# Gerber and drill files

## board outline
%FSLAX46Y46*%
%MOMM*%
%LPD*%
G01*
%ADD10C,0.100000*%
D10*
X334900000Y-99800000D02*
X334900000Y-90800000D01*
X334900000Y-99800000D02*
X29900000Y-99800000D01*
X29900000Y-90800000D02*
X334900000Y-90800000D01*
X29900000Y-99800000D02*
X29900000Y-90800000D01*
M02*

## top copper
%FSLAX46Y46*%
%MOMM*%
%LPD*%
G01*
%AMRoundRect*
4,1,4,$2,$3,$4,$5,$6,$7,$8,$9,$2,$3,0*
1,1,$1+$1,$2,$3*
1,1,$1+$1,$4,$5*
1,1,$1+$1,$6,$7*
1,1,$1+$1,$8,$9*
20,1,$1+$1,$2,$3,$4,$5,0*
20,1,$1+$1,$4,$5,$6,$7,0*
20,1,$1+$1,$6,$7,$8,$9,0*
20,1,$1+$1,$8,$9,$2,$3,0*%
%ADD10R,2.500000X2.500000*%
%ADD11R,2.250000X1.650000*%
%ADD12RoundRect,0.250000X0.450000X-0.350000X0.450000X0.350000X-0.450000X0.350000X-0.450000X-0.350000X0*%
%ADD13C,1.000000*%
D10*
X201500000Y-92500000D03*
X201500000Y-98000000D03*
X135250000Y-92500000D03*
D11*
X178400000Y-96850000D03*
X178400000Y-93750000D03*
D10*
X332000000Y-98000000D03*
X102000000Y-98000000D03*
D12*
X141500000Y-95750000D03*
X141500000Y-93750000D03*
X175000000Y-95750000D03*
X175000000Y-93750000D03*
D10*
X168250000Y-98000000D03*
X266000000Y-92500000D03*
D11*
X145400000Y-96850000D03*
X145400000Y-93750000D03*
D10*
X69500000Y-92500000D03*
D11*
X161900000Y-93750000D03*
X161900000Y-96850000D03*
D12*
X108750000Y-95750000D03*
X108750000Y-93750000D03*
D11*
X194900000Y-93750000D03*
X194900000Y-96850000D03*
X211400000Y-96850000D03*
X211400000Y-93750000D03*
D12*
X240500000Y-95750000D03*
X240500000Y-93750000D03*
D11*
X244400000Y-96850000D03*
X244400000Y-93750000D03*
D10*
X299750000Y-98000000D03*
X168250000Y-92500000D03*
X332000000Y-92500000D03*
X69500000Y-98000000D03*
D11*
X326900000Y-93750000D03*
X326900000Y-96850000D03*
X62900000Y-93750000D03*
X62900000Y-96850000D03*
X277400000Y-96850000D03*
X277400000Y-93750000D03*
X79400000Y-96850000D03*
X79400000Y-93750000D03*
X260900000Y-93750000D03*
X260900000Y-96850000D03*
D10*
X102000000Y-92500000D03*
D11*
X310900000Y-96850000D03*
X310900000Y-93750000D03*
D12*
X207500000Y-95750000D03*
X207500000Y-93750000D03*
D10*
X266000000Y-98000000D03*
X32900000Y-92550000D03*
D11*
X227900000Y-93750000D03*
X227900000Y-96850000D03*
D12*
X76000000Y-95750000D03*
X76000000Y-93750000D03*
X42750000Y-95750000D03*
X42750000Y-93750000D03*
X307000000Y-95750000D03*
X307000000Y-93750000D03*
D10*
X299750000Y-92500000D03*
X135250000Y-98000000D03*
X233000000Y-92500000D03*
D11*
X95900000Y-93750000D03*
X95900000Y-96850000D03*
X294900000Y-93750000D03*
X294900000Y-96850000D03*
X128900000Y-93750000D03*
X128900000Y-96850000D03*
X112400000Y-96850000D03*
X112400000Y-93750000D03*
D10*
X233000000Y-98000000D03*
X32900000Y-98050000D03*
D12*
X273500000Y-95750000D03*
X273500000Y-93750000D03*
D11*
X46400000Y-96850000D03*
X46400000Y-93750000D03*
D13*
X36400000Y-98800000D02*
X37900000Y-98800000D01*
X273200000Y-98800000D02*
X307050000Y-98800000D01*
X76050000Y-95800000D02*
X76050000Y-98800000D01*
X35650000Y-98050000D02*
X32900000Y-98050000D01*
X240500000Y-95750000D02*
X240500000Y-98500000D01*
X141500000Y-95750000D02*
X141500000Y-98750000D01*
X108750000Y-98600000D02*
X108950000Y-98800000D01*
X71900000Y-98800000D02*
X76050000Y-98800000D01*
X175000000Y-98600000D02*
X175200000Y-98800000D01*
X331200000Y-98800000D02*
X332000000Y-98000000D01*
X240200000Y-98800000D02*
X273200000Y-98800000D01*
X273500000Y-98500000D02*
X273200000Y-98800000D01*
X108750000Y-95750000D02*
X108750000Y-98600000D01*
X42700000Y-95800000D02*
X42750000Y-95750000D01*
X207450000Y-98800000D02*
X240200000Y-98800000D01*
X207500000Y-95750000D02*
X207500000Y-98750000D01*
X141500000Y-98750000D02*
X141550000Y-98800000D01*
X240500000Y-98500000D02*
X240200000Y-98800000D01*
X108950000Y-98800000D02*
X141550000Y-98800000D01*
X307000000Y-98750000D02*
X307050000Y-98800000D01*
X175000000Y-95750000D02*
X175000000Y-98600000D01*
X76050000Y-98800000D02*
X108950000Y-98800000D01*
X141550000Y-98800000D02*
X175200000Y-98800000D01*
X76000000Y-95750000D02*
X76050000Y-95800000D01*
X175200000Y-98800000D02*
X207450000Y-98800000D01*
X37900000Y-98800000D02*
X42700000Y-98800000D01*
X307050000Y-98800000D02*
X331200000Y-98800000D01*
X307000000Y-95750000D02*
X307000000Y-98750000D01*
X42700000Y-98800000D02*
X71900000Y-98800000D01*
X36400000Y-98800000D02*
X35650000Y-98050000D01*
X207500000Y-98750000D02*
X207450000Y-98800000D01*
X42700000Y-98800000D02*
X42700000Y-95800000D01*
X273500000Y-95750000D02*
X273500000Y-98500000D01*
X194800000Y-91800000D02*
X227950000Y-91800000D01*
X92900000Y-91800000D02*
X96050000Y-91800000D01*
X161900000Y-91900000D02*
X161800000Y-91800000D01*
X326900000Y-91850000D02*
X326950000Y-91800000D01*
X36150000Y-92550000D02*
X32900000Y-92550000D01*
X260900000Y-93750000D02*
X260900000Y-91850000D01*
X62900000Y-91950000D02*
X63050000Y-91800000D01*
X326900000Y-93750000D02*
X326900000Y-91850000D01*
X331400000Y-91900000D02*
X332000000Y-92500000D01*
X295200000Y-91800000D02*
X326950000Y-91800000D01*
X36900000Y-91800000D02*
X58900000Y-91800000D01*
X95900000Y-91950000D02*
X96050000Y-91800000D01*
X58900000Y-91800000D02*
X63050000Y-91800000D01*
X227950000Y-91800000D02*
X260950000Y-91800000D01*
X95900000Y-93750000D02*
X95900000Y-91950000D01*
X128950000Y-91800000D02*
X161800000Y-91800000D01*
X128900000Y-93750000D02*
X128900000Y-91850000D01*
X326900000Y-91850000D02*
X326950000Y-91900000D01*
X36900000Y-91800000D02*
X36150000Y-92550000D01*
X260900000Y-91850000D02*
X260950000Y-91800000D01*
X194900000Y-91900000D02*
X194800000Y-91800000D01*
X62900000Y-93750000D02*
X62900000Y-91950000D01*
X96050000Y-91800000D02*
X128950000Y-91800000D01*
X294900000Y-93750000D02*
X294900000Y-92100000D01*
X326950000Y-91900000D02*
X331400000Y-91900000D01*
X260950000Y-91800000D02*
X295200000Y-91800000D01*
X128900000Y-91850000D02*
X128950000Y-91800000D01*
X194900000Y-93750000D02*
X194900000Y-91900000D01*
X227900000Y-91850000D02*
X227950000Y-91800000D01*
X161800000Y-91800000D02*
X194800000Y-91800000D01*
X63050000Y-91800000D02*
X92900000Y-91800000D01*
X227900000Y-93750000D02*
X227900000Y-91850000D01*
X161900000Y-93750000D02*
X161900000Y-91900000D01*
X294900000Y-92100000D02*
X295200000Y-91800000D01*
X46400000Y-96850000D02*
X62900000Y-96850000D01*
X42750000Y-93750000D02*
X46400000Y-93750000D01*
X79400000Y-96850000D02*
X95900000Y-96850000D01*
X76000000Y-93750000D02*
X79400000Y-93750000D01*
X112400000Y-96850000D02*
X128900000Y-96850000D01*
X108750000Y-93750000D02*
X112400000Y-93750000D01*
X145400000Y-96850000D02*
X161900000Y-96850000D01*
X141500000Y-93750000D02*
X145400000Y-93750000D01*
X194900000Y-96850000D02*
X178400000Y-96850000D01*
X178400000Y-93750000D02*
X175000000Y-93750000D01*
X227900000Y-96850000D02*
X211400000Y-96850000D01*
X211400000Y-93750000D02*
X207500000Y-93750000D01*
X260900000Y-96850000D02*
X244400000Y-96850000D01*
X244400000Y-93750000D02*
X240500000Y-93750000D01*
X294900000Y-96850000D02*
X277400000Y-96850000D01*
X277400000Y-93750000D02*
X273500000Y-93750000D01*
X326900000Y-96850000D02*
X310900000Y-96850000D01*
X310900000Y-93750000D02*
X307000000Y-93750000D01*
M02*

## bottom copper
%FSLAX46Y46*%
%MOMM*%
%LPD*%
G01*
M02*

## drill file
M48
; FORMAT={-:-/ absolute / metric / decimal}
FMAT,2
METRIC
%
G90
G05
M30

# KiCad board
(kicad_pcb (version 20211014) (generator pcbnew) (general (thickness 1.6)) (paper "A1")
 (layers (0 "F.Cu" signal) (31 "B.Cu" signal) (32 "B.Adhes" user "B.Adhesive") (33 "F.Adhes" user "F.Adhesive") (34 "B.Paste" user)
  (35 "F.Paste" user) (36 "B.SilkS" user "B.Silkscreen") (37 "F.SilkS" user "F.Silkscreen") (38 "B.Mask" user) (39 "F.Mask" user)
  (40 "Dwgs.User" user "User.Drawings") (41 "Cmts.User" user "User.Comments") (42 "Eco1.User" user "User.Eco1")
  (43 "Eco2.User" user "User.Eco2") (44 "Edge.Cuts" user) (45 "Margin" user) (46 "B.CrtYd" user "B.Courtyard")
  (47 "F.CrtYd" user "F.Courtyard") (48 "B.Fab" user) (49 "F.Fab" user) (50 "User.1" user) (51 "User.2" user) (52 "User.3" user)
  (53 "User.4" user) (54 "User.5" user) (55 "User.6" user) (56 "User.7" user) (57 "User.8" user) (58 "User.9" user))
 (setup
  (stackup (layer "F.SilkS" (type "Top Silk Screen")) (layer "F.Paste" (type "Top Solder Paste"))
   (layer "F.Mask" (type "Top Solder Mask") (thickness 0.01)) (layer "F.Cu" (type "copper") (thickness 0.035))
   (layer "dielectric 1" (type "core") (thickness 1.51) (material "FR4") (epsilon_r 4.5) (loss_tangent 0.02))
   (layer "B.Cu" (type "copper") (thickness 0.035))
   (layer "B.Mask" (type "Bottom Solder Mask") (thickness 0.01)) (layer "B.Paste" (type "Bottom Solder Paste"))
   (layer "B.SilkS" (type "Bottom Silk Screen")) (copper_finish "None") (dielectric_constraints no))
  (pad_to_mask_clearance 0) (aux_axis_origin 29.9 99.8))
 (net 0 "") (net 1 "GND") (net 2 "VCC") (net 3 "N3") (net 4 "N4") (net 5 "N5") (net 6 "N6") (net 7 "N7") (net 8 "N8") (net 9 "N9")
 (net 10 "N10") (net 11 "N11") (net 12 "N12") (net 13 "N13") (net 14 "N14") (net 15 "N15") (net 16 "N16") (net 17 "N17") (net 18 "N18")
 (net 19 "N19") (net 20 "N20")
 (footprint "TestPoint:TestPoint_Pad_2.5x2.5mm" (layer "F.Cu") (at 201.5 92.5)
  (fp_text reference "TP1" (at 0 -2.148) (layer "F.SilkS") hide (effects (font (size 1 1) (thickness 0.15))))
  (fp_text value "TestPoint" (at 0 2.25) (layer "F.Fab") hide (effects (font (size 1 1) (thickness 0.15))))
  (pad "1" smd rect (at 0 0) (size 2.5 2.5) (layers "F.Cu" "F.Mask") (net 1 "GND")))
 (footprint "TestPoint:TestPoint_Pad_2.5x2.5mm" (layer "F.Cu") (at 201.5 98)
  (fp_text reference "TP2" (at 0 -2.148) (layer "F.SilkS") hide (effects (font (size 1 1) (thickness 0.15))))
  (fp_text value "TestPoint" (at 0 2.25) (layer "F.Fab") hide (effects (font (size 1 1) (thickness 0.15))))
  (pad "1" smd rect (at 0 0) (size 2.5 2.5) (layers "F.Cu" "F.Mask") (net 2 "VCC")))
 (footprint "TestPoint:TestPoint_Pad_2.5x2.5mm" (layer "F.Cu") (at 135.25 92.5)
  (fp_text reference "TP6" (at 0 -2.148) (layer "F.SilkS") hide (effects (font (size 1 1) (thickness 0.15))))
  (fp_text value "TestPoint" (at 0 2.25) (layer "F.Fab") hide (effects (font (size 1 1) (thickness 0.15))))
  (pad "1" smd rect (at 0 0) (size 2.5 2.5) (layers "F.Cu" "F.Mask") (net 1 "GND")))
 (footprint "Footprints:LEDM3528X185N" (layer "F.Cu") (at 178.4 95.3 90)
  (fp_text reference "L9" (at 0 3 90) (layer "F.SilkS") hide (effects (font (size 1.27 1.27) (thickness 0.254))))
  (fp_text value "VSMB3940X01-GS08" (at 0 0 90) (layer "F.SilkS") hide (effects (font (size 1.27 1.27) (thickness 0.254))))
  (pad "1" smd rect (at -1.55 0 90) (size 1.65 2.25) (layers "F.Cu" "F.Paste" "F.Mask") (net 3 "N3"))
  (pad "2" smd rect (at 1.55 0 90) (size 1.65 2.25) (layers "F.Cu" "F.Paste" "F.Mask") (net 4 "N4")))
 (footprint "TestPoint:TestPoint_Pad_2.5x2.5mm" (layer "F.Cu") (at 332 98)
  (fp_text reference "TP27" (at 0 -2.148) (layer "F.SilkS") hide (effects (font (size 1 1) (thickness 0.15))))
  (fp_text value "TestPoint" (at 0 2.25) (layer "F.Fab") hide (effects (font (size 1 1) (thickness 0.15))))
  (pad "1" smd rect (at 0 0) (size 2.5 2.5) (layers "F.Cu" "F.Mask") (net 2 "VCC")))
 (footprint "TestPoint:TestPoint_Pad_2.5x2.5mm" (layer "F.Cu") (at 102 98)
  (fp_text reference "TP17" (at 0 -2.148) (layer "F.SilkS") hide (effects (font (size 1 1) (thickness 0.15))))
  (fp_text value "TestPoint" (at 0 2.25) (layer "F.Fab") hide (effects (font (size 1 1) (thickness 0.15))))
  (pad "1" smd rect (at 0 0) (size 2.5 2.5) (layers "F.Cu" "F.Mask") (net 2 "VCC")))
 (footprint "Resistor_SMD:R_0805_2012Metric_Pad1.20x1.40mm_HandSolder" (layer "F.Cu") (at 141.5 94.75 90)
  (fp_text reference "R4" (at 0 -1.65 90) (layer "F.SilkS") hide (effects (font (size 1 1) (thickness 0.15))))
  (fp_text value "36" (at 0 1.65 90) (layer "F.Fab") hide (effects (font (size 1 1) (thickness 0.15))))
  (pad "1" smd roundrect (at -1 0 90) (size 1.2 1.4) (layers "F.Cu" "F.Paste" "F.Mask") (roundrect_rratio 0.2083333333) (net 2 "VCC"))
  (pad "2" smd roundrect (at 1 0 90) (size 1.2 1.4) (layers "F.Cu" "F.Paste" "F.Mask") (roundrect_rratio 0.2083333333) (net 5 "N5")))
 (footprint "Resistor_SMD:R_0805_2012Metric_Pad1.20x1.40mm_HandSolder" (layer "F.Cu") (at 175 94.75 90)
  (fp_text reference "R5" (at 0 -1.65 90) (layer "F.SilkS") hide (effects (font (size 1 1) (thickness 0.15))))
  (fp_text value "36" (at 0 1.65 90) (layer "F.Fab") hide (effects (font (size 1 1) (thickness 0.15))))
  (pad "1" smd roundrect (at -1 0 90) (size 1.2 1.4) (layers "F.Cu" "F.Paste" "F.Mask") (roundrect_rratio 0.2083333333) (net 2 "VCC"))
  (pad "2" smd roundrect (at 1 0 90) (size 1.2 1.4) (layers "F.Cu" "F.Paste" "F.Mask") (roundrect_rratio 0.2083333333) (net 4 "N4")))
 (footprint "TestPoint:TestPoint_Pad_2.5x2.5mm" (layer "F.Cu") (at 168.25 98)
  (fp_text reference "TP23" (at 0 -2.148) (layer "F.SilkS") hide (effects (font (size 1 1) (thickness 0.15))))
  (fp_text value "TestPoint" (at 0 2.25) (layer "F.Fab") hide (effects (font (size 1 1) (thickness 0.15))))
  (pad "1" smd rect (at 0 0) (size 2.5 2.5) (layers "F.Cu" "F.Mask") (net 2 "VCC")))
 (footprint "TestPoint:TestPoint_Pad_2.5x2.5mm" (layer "F.Cu") (at 266 92.5)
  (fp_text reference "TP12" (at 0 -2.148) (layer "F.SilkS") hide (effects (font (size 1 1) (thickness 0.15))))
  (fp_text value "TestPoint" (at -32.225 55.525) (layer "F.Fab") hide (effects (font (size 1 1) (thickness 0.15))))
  (pad "1" smd rect (at 0 0) (size 2.5 2.5) (layers "F.Cu" "F.Mask") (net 1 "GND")))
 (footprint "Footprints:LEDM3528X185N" (layer "F.Cu") (at 145.4 95.3 90)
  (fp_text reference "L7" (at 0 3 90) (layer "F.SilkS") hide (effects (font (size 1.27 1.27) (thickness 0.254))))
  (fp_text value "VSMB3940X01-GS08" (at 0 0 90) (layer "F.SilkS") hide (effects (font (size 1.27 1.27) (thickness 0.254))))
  (pad "1" smd rect (at -1.55 0 90) (size 1.65 2.25) (layers "F.Cu" "F.Paste" "F.Mask") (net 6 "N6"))
  (pad "2" smd rect (at 1.55 0 90) (size 1.65 2.25) (layers "F.Cu" "F.Paste" "F.Mask") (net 5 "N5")))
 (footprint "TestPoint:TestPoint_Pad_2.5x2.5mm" (layer "F.Cu") (at 69.5 92.5)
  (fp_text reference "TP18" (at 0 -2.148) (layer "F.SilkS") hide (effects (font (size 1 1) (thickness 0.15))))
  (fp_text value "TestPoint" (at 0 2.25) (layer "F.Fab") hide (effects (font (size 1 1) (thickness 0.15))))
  (pad "1" smd rect (at 0 0) (size 2.5 2.5) (layers "F.Cu" "F.Mask") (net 1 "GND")))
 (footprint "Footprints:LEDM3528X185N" (layer "F.Cu") (at 161.9 95.3 -90)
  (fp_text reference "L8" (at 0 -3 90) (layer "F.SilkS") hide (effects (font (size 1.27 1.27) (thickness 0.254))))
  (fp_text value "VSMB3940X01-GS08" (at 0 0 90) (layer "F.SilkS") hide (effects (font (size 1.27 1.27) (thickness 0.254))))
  (pad "1" smd rect (at -1.55 0 270) (size 1.65 2.25) (layers "F.Cu" "F.Paste" "F.Mask") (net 1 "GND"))
  (pad "2" smd rect (at 1.55 0 270) (size 1.65 2.25) (layers "F.Cu" "F.Paste" "F.Mask") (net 6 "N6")))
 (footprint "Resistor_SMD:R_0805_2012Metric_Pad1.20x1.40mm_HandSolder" (layer "F.Cu") (at 108.75 94.75 90)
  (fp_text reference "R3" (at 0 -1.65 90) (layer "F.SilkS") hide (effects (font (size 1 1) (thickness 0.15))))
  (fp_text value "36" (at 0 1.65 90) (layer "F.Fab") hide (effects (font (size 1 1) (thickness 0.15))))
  (pad "1" smd roundrect (at -1 0 90) (size 1.2 1.4) (layers "F.Cu" "F.Paste" "F.Mask") (roundrect_rratio 0.2083333333) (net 2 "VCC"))
  (pad "2" smd roundrect (at 1 0 90) (size 1.2 1.4) (layers "F.Cu" "F.Paste" "F.Mask") (roundrect_rratio 0.2083333333) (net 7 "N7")))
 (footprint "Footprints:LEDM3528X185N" (layer "F.Cu") (at 194.9 95.3 -90)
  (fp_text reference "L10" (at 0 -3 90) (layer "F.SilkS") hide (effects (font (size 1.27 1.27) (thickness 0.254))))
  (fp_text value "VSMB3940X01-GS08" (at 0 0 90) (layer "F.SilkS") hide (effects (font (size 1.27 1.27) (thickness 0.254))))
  (pad "1" smd rect (at -1.55 0 270) (size 1.65 2.25) (layers "F.Cu" "F.Paste" "F.Mask") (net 1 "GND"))
  (pad "2" smd rect (at 1.55 0 270) (size 1.65 2.25) (layers "F.Cu" "F.Paste" "F.Mask") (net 3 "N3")))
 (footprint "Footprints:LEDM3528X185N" (layer "F.Cu") (at 211.4 95.3 90)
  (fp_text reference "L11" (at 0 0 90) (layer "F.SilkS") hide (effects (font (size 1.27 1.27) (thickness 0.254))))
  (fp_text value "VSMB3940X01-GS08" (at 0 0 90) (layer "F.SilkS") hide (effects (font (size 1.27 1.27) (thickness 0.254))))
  (pad "1" smd rect (at -1.55 0 90) (size 1.65 2.25) (layers "F.Cu" "F.Paste" "F.Mask") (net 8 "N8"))
  (pad "2" smd rect (at 1.55 0 90) (size 1.65 2.25) (layers "F.Cu" "F.Paste" "F.Mask") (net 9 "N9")))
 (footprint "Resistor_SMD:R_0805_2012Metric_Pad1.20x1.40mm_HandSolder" (layer "F.Cu") (at 240.5 94.75 90)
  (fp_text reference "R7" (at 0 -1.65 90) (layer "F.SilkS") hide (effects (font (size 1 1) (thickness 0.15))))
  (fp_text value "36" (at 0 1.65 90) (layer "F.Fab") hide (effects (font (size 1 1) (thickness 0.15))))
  (pad "1" smd roundrect (at -1 0 90) (size 1.2 1.4) (layers "F.Cu" "F.Paste" "F.Mask") (roundrect_rratio 0.2083333333) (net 2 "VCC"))
  (pad "2" smd roundrect (at 1 0 90) (size 1.2 1.4) (layers "F.Cu" "F.Paste" "F.Mask") (roundrect_rratio 0.2083333333) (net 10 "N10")))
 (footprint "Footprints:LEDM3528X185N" (layer "F.Cu") (at 244.4 95.3 90)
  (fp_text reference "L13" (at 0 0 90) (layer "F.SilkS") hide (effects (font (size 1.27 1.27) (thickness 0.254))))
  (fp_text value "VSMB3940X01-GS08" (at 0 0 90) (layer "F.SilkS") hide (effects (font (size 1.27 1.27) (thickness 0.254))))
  (pad "1" smd rect (at -1.55 0 90) (size 1.65 2.25) (layers "F.Cu" "F.Paste" "F.Mask") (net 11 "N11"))
  (pad "2" smd rect (at 1.55 0 90) (size 1.65 2.25) (layers "F.Cu" "F.Paste" "F.Mask") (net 10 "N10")))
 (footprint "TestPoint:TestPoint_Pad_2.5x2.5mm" (layer "F.Cu") (at 299.75 98)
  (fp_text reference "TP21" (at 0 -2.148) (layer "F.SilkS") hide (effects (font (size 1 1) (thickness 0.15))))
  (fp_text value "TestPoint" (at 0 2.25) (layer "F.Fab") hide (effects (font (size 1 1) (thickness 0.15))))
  (pad "1" smd rect (at 0 0) (size 2.5 2.5) (layers "F.Cu" "F.Mask") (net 2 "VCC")))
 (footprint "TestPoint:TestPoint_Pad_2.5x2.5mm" (layer "F.Cu") (at 168.25 92.5)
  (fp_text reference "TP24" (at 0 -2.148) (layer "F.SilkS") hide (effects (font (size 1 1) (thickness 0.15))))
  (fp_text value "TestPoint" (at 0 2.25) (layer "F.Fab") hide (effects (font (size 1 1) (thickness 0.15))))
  (pad "1" smd rect (at 0 0) (size 2.5 2.5) (layers "F.Cu" "F.Mask") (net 1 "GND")))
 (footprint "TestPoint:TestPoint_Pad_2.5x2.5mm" (layer "F.Cu") (at 332 92.5)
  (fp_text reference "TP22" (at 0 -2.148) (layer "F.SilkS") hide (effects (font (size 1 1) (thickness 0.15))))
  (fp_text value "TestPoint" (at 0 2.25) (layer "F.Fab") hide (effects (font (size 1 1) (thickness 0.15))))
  (pad "1" smd rect (at 0 0) (size 2.5 2.5) (layers "F.Cu" "F.Mask") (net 1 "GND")))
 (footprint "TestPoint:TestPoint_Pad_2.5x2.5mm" (layer "F.Cu") (at 69.5 98)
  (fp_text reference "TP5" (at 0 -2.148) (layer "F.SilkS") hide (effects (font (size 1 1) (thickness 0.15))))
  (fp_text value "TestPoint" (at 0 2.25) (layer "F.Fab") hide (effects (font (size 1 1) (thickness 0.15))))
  (pad "1" smd rect (at 0 0) (size 2.5 2.5) (layers "F.Cu" "F.Mask") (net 2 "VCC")))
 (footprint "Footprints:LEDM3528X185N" (layer "F.Cu") (at 326.9 95.3 -90)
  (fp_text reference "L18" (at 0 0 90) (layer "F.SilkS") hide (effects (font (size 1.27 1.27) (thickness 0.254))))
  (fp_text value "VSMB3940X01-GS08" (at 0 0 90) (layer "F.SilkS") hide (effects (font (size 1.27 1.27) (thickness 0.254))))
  (pad "1" smd rect (at -1.55 0 270) (size 1.65 2.25) (layers "F.Cu" "F.Paste" "F.Mask") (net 1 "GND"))
  (pad "2" smd rect (at 1.55 0 270) (size 1.65 2.25) (layers "F.Cu" "F.Paste" "F.Mask") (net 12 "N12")))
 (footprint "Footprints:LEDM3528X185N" (layer "F.Cu") (at 62.9 95.3 -90)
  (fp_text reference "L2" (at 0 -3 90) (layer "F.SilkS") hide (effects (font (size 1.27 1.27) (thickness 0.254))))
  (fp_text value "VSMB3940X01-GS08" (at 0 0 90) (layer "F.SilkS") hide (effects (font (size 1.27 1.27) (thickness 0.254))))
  (pad "1" smd rect (at -1.55 0 270) (size 1.65 2.25) (layers "F.Cu" "F.Paste" "F.Mask") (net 1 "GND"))
  (pad "2" smd rect (at 1.55 0 270) (size 1.65 2.25) (layers "F.Cu" "F.Paste" "F.Mask") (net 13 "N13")))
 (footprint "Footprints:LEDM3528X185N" (layer "F.Cu") (at 277.4 95.3 90)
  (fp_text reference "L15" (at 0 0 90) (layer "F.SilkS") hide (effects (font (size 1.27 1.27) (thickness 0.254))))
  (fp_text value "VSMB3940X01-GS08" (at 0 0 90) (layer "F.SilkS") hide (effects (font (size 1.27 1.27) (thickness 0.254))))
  (pad "1" smd rect (at -1.55 0 90) (size 1.65 2.25) (layers "F.Cu" "F.Paste" "F.Mask") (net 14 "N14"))
  (pad "2" smd rect (at 1.55 0 90) (size 1.65 2.25) (layers "F.Cu" "F.Paste" "F.Mask") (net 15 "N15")))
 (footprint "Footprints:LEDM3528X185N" (layer "F.Cu") (at 79.4 95.3 90)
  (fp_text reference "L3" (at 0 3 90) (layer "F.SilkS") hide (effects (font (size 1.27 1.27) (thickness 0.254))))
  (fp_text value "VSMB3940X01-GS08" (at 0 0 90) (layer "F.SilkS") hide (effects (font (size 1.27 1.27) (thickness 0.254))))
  (pad "1" smd rect (at -1.55 0 90) (size 1.65 2.25) (layers "F.Cu" "F.Paste" "F.Mask") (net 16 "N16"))
  (pad "2" smd rect (at 1.55 0 90) (size 1.65 2.25) (layers "F.Cu" "F.Paste" "F.Mask") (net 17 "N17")))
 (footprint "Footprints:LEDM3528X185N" (layer "F.Cu") (at 260.9 95.3 -90)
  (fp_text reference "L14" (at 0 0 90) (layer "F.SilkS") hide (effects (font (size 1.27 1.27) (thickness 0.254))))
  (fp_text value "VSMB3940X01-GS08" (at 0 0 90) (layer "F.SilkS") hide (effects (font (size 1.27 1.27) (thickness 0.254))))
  (pad "1" smd rect (at -1.55 0 270) (size 1.65 2.25) (layers "F.Cu" "F.Paste" "F.Mask") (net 1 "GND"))
  (pad "2" smd rect (at 1.55 0 270) (size 1.65 2.25) (layers "F.Cu" "F.Paste" "F.Mask") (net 11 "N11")))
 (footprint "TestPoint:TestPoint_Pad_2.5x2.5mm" (layer "F.Cu") (at 102 92.5)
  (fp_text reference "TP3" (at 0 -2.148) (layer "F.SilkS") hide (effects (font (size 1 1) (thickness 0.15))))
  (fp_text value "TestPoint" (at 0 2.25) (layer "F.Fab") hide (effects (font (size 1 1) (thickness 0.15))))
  (pad "1" smd rect (at 0 0) (size 2.5 2.5) (layers "F.Cu" "F.Mask") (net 1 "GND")))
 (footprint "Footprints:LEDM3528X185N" (layer "F.Cu") (at 310.9 95.3 90)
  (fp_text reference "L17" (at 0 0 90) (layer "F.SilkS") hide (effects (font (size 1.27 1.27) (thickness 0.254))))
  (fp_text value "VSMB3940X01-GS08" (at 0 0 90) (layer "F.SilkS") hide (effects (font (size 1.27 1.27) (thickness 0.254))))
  (pad "1" smd rect (at -1.55 0 90) (size 1.65 2.25) (layers "F.Cu" "F.Paste" "F.Mask") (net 12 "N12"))
  (pad "2" smd rect (at 1.55 0 90) (size 1.65 2.25) (layers "F.Cu" "F.Paste" "F.Mask") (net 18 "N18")))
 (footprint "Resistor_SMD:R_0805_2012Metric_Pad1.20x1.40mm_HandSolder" (layer "F.Cu") (at 207.5 94.75 90)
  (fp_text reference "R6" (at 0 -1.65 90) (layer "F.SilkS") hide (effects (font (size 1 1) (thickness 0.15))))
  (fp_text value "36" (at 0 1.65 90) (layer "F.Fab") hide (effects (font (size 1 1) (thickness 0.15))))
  (pad "1" smd roundrect (at -1 0 90) (size 1.2 1.4) (layers "F.Cu" "F.Paste" "F.Mask") (roundrect_rratio 0.2083333333) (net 2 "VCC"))
  (pad "2" smd roundrect (at 1 0 90) (size 1.2 1.4) (layers "F.Cu" "F.Paste" "F.Mask") (roundrect_rratio 0.2083333333) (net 9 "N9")))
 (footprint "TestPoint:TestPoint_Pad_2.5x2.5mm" (layer "F.Cu") (at 266 98)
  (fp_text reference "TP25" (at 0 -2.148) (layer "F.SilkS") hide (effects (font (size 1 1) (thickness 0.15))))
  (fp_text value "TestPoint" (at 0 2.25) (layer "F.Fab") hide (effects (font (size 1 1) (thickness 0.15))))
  (pad "1" smd rect (at 0 0) (size 2.5 2.5) (layers "F.Cu" "F.Mask") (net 2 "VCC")))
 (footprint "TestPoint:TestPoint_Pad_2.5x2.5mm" (layer "F.Cu") (at 32.9 92.55)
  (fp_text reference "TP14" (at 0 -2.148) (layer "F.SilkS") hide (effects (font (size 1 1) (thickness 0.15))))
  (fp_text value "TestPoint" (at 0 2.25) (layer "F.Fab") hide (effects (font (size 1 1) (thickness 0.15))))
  (pad "1" smd rect (at 0 0) (size 2.5 2.5) (layers "F.Cu" "F.Mask") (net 1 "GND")))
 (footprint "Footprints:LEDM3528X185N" (layer "F.Cu") (at 227.9 95.3 -90)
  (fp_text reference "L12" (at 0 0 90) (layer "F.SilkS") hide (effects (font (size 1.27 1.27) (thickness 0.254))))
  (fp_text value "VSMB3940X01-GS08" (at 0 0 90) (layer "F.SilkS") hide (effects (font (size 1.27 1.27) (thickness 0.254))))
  (pad "1" smd rect (at -1.55 0 270) (size 1.65 2.25) (layers "F.Cu" "F.Paste" "F.Mask") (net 1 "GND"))
  (pad "2" smd rect (at 1.55 0 270) (size 1.65 2.25) (layers "F.Cu" "F.Paste" "F.Mask") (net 8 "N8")))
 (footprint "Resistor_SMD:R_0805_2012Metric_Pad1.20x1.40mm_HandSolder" (layer "F.Cu") (at 76 94.75 90)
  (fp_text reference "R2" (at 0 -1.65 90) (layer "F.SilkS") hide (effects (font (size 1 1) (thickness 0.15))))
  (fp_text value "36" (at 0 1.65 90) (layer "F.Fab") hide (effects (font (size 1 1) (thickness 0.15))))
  (pad "1" smd roundrect (at -1 0 90) (size 1.2 1.4) (layers "F.Cu" "F.Paste" "F.Mask") (roundrect_rratio 0.2083333333) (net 2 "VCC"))
  (pad "2" smd roundrect (at 1 0 90) (size 1.2 1.4) (layers "F.Cu" "F.Paste" "F.Mask") (roundrect_rratio 0.2083333333) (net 17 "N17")))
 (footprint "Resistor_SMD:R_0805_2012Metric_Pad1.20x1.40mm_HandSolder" (layer "F.Cu") (at 42.75 94.75 90)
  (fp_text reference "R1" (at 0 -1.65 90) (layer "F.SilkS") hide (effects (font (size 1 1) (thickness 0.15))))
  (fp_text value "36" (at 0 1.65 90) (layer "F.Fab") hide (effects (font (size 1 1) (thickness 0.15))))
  (pad "1" smd roundrect (at -1 0 90) (size 1.2 1.4) (layers "F.Cu" "F.Paste" "F.Mask") (roundrect_rratio 0.2083333333) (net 2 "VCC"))
  (pad "2" smd roundrect (at 1 0 90) (size 1.2 1.4) (layers "F.Cu" "F.Paste" "F.Mask") (roundrect_rratio 0.2083333333) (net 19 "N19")))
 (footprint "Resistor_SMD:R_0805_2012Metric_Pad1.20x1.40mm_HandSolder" (layer "F.Cu") (at 307 94.75 90)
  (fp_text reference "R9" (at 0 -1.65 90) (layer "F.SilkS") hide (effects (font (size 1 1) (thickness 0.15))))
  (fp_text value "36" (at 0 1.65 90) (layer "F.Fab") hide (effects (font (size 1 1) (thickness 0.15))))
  (pad "1" smd roundrect (at -1 0 90) (size 1.2 1.4) (layers "F.Cu" "F.Paste" "F.Mask") (roundrect_rratio 0.2083333333) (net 2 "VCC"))
  (pad "2" smd roundrect (at 1 0 90) (size 1.2 1.4) (layers "F.Cu" "F.Paste" "F.Mask") (roundrect_rratio 0.2083333333) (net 18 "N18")))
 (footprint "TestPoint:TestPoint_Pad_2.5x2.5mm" (layer "F.Cu") (at 299.75 92.5)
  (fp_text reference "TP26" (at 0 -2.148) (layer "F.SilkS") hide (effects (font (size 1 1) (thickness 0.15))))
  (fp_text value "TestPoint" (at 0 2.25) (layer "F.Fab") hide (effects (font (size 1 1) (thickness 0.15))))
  (pad "1" smd rect (at 0 0) (size 2.5 2.5) (layers "F.Cu" "F.Mask") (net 1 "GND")))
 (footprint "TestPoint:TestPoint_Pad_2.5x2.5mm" (layer "F.Cu") (at 135.25 98)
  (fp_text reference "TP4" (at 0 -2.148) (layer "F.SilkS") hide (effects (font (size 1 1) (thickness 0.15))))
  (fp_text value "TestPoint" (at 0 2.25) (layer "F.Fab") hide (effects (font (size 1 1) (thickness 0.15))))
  (pad "1" smd rect (at 0 0) (size 2.5 2.5) (layers "F.Cu" "F.Mask") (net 2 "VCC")))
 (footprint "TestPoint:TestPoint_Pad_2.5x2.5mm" (layer "F.Cu") (at 233 92.5)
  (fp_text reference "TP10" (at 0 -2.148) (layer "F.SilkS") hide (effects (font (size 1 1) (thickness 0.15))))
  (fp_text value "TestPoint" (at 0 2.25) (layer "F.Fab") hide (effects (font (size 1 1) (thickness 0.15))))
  (pad "1" smd rect (at 0 0) (size 2.5 2.5) (layers "F.Cu" "F.Mask") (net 1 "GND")))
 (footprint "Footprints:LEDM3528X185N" (layer "F.Cu") (at 95.9 95.3 -90)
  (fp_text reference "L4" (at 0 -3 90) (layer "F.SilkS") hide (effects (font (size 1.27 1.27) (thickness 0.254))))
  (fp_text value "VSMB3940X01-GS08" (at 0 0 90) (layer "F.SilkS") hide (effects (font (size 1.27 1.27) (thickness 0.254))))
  (pad "1" smd rect (at -1.55 0 270) (size 1.65 2.25) (layers "F.Cu" "F.Paste" "F.Mask") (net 1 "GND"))
  (pad "2" smd rect (at 1.55 0 270) (size 1.65 2.25) (layers "F.Cu" "F.Paste" "F.Mask") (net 16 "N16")))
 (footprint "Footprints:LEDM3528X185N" (layer "F.Cu") (at 294.9 95.3 -90)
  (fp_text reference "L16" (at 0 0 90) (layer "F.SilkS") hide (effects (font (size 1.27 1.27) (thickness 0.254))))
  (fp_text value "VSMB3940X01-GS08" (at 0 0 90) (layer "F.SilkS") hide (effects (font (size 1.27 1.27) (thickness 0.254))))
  (pad "1" smd rect (at -1.55 0 270) (size 1.65 2.25) (layers "F.Cu" "F.Paste" "F.Mask") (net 1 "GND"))
  (pad "2" smd rect (at 1.55 0 270) (size 1.65 2.25) (layers "F.Cu" "F.Paste" "F.Mask") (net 14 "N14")))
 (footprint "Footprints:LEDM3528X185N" (layer "F.Cu") (at 128.9 95.3 -90)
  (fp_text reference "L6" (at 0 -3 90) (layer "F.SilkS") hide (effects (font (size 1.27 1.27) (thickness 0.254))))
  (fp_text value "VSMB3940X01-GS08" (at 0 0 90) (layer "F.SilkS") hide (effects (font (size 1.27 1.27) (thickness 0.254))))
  (pad "1" smd rect (at -1.55 0 270) (size 1.65 2.25) (layers "F.Cu" "F.Paste" "F.Mask") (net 1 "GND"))
  (pad "2" smd rect (at 1.55 0 270) (size 1.65 2.25) (layers "F.Cu" "F.Paste" "F.Mask") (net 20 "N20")))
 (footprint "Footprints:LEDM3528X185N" (layer "F.Cu") (at 112.4 95.3 90)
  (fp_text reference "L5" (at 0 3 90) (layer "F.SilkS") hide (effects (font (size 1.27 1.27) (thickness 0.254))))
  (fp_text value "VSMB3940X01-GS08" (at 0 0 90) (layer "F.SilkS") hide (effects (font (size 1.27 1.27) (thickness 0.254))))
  (pad "1" smd rect (at -1.55 0 90) (size 1.65 2.25) (layers "F.Cu" "F.Paste" "F.Mask") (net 20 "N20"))
  (pad "2" smd rect (at 1.55 0 90) (size 1.65 2.25) (layers "F.Cu" "F.Paste" "F.Mask") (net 7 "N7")))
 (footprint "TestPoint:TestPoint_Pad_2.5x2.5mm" (layer "F.Cu") (at 233 98)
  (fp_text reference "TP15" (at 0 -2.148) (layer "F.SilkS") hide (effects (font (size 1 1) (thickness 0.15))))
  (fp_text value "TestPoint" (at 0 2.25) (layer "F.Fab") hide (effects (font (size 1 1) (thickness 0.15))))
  (pad "1" smd rect (at 0 0) (size 2.5 2.5) (layers "F.Cu" "F.Mask") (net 2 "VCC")))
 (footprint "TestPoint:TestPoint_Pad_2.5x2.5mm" (layer "F.Cu") (at 32.9 98.05)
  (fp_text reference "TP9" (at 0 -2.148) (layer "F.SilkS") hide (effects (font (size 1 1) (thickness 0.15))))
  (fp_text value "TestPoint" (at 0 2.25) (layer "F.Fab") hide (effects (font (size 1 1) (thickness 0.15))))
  (pad "1" smd rect (at 0 0) (size 2.5 2.5) (layers "F.Cu" "F.Mask") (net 2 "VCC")))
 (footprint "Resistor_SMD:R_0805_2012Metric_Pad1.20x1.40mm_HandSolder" (layer "F.Cu") (at 273.5 94.75 90)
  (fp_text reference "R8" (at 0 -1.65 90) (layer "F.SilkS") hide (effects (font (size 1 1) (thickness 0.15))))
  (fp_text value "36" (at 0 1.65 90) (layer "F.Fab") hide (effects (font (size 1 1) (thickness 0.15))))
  (pad "1" smd roundrect (at -1 0 90) (size 1.2 1.4) (layers "F.Cu" "F.Paste" "F.Mask") (roundrect_rratio 0.2083333333) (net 2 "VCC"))
  (pad "2" smd roundrect (at 1 0 90) (size 1.2 1.4) (layers "F.Cu" "F.Paste" "F.Mask") (roundrect_rratio 0.2083333333) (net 15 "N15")))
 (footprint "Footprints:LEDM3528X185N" (layer "F.Cu") (at 46.4 95.3 90)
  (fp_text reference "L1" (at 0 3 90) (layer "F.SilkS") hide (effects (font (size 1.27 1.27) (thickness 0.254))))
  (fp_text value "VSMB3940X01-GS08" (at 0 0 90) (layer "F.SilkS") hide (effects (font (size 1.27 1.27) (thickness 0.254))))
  (pad "1" smd rect (at -1.55 0 90) (size 1.65 2.25) (layers "F.Cu" "F.Paste" "F.Mask") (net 13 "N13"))
  (pad "2" smd rect (at 1.55 0 90) (size 1.65 2.25) (layers "F.Cu" "F.Paste" "F.Mask") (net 19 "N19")))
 (gr_line (start 334.9 99.8) (end 334.9 90.8) (layer "Edge.Cuts") (width 0.1))
 (gr_line (start 334.9 99.8) (end 29.9 99.8) (layer "Edge.Cuts") (width 0.1))
 (gr_line (start 29.9 90.8) (end 334.9 90.8) (layer "Edge.Cuts") (width 0.1))
 (gr_line (start 29.9 99.8) (end 29.9 90.8) (layer "Edge.Cuts") (width 0.1))
 (segment (start 36.4 98.8) (end 37.9 98.8) (width 1) (layer "F.Cu") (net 2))
 (segment (start 273.2 98.8) (end 307.05 98.8) (width 1) (layer "F.Cu") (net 2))
 (segment (start 76.05 95.8) (end 76.05 98.8) (width 1) (layer "F.Cu") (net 2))
 (segment (start 35.65 98.05) (end 32.9 98.05) (width 1) (layer "F.Cu") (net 2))
 (segment (start 240.5 95.75) (end 240.5 98.5) (width 1) (layer "F.Cu") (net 2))
 (segment (start 141.5 95.75) (end 141.5 98.75) (width 1) (layer "F.Cu") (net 2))
 (segment (start 108.75 98.6) (end 108.95 98.8) (width 1) (layer "F.Cu") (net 2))
 (segment (start 71.9 98.8) (end 76.05 98.8) (width 1) (layer "F.Cu") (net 2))
 (segment (start 175 98.6) (end 175.2 98.8) (width 1) (layer "F.Cu") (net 2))
 (segment (start 331.2 98.8) (end 332 98) (width 1) (layer "F.Cu") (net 2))
 (segment (start 240.2 98.8) (end 273.2 98.8) (width 1) (layer "F.Cu") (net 2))
 (segment (start 273.5 98.5) (end 273.2 98.8) (width 1) (layer "F.Cu") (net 2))
 (segment (start 108.75 95.75) (end 108.75 98.6) (width 1) (layer "F.Cu") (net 2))
 (segment (start 42.7 95.8) (end 42.75 95.75) (width 1) (layer "F.Cu") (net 2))
 (segment (start 207.45 98.8) (end 240.2 98.8) (width 1) (layer "F.Cu") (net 2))
 (segment (start 207.5 95.75) (end 207.5 98.75) (width 1) (layer "F.Cu") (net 2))
 (segment (start 141.5 98.75) (end 141.55 98.8) (width 1) (layer "F.Cu") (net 2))
 (segment (start 240.5 98.5) (end 240.2 98.8) (width 1) (layer "F.Cu") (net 2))
 (segment (start 108.95 98.8) (end 141.55 98.8) (width 1) (layer "F.Cu") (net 2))
 (segment (start 307 98.75) (end 307.05 98.8) (width 1) (layer "F.Cu") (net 2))
 (segment (start 175 95.75) (end 175 98.6) (width 1) (layer "F.Cu") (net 2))
 (segment (start 76.05 98.8) (end 108.95 98.8) (width 1) (layer "F.Cu") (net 2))
 (segment (start 141.55 98.8) (end 175.2 98.8) (width 1) (layer "F.Cu") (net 2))
 (segment (start 76 95.75) (end 76.05 95.8) (width 1) (layer "F.Cu") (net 2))
 (segment (start 175.2 98.8) (end 207.45 98.8) (width 1) (layer "F.Cu") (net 2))
 (segment (start 37.9 98.8) (end 42.7 98.8) (width 1) (layer "F.Cu") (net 2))
 (segment (start 307.05 98.8) (end 331.2 98.8) (width 1) (layer "F.Cu") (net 2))
 (segment (start 307 95.75) (end 307 98.75) (width 1) (layer "F.Cu") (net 2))
 (segment (start 42.7 98.8) (end 71.9 98.8) (width 1) (layer "F.Cu") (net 2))
 (segment (start 36.4 98.8) (end 35.65 98.05) (width 1) (layer "F.Cu") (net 2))
 (segment (start 207.5 98.75) (end 207.45 98.8) (width 1) (layer "F.Cu") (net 2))
 (segment (start 42.7 98.8) (end 42.7 95.8) (width 1) (layer "F.Cu") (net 2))
 (segment (start 273.5 95.75) (end 273.5 98.5) (width 1) (layer "F.Cu") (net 2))
 (segment (start 194.8 91.8) (end 227.95 91.8) (width 1) (layer "F.Cu") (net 1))
 (segment (start 92.9 91.8) (end 96.05 91.8) (width 1) (layer "F.Cu") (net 1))
 (segment (start 161.9 91.9) (end 161.8 91.8) (width 1) (layer "F.Cu") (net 1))
 (segment (start 326.9 91.85) (end 326.95 91.8) (width 1) (layer "F.Cu") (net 1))
 (segment (start 36.15 92.55) (end 32.9 92.55) (width 1) (layer "F.Cu") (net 1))
 (segment (start 260.9 93.75) (end 260.9 91.85) (width 1) (layer "F.Cu") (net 1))
 (segment (start 62.9 91.95) (end 63.05 91.8) (width 1) (layer "F.Cu") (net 1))
 (segment (start 326.9 93.75) (end 326.9 91.85) (width 1) (layer "F.Cu") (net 1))
 (segment (start 331.4 91.9) (end 332 92.5) (width 1) (layer "F.Cu") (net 1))
 (segment (start 295.2 91.8) (end 326.95 91.8) (width 1) (layer "F.Cu") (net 1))
 (segment (start 36.9 91.8) (end 58.9 91.8) (width 1) (layer "F.Cu") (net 1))
 (segment (start 95.9 91.95) (end 96.05 91.8) (width 1) (layer "F.Cu") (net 1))
 (segment (start 58.9 91.8) (end 63.05 91.8) (width 1) (layer "F.Cu") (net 1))
 (segment (start 227.95 91.8) (end 260.95 91.8) (width 1) (layer "F.Cu") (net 1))
 (segment (start 95.9 93.75) (end 95.9 91.95) (width 1) (layer "F.Cu") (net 1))
 (segment (start 128.95 91.8) (end 161.8 91.8) (width 1) (layer "F.Cu") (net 1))
 (segment (start 128.9 93.75) (end 128.9 91.85) (width 1) (layer "F.Cu") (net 1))
 (segment (start 326.9 91.85) (end 326.95 91.9) (width 1) (layer "F.Cu") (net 1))
 (segment (start 36.9 91.8) (end 36.15 92.55) (width 1) (layer "F.Cu") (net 1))
 (segment (start 260.9 91.85) (end 260.95 91.8) (width 1) (layer "F.Cu") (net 1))
 (segment (start 194.9 91.9) (end 194.8 91.8) (width 1) (layer "F.Cu") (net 1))
 (segment (start 62.9 93.75) (end 62.9 91.95) (width 1) (layer "F.Cu") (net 1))
 (segment (start 96.05 91.8) (end 128.95 91.8) (width 1) (layer "F.Cu") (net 1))
 (segment (start 294.9 93.75) (end 294.9 92.1) (width 1) (layer "F.Cu") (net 1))
 (segment (start 326.95 91.9) (end 331.4 91.9) (width 1) (layer "F.Cu") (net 1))
 (segment (start 260.95 91.8) (end 295.2 91.8) (width 1) (layer "F.Cu") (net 1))
 (segment (start 128.9 91.85) (end 128.95 91.8) (width 1) (layer "F.Cu") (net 1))
 (segment (start 194.9 93.75) (end 194.9 91.9) (width 1) (layer "F.Cu") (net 1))
 (segment (start 227.9 91.85) (end 227.95 91.8) (width 1) (layer "F.Cu") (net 1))
 (segment (start 161.8 91.8) (end 194.8 91.8) (width 1) (layer "F.Cu") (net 1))
 (segment (start 63.05 91.8) (end 92.9 91.8) (width 1) (layer "F.Cu") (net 1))
 (segment (start 227.9 93.75) (end 227.9 91.85) (width 1) (layer "F.Cu") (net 1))
 (segment (start 161.9 93.75) (end 161.9 91.9) (width 1) (layer "F.Cu") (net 1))
 (segment (start 294.9 92.1) (end 295.2 91.8) (width 1) (layer "F.Cu") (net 1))
 (segment (start 46.4 96.85) (end 62.9 96.85) (width 1) (layer "F.Cu") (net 13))
 (segment (start 42.75 93.75) (end 46.4 93.75) (width 1) (layer "F.Cu") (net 19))
 (segment (start 79.4 96.85) (end 95.9 96.85) (width 1) (layer "F.Cu") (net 16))
 (segment (start 76 93.75) (end 79.4 93.75) (width 1) (layer "F.Cu") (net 17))
 (segment (start 112.4 96.85) (end 128.9 96.85) (width 1) (layer "F.Cu") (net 20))
 (segment (start 108.75 93.75) (end 112.4 93.75) (width 1) (layer "F.Cu") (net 7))
 (segment (start 145.4 96.85) (end 161.9 96.85) (width 1) (layer "F.Cu") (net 6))
 (segment (start 141.5 93.75) (end 145.4 93.75) (width 1) (layer "F.Cu") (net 5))
 (segment (start 194.9 96.85) (end 178.4 96.85) (width 1) (layer "F.Cu") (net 3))
 (segment (start 178.4 93.75) (end 175 93.75) (width 1) (layer "F.Cu") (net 4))
 (segment (start 227.9 96.85) (end 211.4 96.85) (width 1) (layer "F.Cu") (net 8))
 (segment (start 211.4 93.75) (end 207.5 93.75) (width 1) (layer "F.Cu") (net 9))
 (segment (start 260.9 96.85) (end 244.4 96.85) (width 1) (layer "F.Cu") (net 11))
 (segment (start 244.4 93.75) (end 240.5 93.75) (width 1) (layer "F.Cu") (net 10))
 (segment (start 294.9 96.85) (end 277.4 96.85) (width 1) (layer "F.Cu") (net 14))
 (segment (start 277.4 93.75) (end 273.5 93.75) (width 1) (layer "F.Cu") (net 15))
 (segment (start 326.9 96.85) (end 310.9 96.85) (width 1) (layer "F.Cu") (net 12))
 (segment (start 310.9 93.75) (end 307 93.75) (width 1) (layer "F.Cu") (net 18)))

